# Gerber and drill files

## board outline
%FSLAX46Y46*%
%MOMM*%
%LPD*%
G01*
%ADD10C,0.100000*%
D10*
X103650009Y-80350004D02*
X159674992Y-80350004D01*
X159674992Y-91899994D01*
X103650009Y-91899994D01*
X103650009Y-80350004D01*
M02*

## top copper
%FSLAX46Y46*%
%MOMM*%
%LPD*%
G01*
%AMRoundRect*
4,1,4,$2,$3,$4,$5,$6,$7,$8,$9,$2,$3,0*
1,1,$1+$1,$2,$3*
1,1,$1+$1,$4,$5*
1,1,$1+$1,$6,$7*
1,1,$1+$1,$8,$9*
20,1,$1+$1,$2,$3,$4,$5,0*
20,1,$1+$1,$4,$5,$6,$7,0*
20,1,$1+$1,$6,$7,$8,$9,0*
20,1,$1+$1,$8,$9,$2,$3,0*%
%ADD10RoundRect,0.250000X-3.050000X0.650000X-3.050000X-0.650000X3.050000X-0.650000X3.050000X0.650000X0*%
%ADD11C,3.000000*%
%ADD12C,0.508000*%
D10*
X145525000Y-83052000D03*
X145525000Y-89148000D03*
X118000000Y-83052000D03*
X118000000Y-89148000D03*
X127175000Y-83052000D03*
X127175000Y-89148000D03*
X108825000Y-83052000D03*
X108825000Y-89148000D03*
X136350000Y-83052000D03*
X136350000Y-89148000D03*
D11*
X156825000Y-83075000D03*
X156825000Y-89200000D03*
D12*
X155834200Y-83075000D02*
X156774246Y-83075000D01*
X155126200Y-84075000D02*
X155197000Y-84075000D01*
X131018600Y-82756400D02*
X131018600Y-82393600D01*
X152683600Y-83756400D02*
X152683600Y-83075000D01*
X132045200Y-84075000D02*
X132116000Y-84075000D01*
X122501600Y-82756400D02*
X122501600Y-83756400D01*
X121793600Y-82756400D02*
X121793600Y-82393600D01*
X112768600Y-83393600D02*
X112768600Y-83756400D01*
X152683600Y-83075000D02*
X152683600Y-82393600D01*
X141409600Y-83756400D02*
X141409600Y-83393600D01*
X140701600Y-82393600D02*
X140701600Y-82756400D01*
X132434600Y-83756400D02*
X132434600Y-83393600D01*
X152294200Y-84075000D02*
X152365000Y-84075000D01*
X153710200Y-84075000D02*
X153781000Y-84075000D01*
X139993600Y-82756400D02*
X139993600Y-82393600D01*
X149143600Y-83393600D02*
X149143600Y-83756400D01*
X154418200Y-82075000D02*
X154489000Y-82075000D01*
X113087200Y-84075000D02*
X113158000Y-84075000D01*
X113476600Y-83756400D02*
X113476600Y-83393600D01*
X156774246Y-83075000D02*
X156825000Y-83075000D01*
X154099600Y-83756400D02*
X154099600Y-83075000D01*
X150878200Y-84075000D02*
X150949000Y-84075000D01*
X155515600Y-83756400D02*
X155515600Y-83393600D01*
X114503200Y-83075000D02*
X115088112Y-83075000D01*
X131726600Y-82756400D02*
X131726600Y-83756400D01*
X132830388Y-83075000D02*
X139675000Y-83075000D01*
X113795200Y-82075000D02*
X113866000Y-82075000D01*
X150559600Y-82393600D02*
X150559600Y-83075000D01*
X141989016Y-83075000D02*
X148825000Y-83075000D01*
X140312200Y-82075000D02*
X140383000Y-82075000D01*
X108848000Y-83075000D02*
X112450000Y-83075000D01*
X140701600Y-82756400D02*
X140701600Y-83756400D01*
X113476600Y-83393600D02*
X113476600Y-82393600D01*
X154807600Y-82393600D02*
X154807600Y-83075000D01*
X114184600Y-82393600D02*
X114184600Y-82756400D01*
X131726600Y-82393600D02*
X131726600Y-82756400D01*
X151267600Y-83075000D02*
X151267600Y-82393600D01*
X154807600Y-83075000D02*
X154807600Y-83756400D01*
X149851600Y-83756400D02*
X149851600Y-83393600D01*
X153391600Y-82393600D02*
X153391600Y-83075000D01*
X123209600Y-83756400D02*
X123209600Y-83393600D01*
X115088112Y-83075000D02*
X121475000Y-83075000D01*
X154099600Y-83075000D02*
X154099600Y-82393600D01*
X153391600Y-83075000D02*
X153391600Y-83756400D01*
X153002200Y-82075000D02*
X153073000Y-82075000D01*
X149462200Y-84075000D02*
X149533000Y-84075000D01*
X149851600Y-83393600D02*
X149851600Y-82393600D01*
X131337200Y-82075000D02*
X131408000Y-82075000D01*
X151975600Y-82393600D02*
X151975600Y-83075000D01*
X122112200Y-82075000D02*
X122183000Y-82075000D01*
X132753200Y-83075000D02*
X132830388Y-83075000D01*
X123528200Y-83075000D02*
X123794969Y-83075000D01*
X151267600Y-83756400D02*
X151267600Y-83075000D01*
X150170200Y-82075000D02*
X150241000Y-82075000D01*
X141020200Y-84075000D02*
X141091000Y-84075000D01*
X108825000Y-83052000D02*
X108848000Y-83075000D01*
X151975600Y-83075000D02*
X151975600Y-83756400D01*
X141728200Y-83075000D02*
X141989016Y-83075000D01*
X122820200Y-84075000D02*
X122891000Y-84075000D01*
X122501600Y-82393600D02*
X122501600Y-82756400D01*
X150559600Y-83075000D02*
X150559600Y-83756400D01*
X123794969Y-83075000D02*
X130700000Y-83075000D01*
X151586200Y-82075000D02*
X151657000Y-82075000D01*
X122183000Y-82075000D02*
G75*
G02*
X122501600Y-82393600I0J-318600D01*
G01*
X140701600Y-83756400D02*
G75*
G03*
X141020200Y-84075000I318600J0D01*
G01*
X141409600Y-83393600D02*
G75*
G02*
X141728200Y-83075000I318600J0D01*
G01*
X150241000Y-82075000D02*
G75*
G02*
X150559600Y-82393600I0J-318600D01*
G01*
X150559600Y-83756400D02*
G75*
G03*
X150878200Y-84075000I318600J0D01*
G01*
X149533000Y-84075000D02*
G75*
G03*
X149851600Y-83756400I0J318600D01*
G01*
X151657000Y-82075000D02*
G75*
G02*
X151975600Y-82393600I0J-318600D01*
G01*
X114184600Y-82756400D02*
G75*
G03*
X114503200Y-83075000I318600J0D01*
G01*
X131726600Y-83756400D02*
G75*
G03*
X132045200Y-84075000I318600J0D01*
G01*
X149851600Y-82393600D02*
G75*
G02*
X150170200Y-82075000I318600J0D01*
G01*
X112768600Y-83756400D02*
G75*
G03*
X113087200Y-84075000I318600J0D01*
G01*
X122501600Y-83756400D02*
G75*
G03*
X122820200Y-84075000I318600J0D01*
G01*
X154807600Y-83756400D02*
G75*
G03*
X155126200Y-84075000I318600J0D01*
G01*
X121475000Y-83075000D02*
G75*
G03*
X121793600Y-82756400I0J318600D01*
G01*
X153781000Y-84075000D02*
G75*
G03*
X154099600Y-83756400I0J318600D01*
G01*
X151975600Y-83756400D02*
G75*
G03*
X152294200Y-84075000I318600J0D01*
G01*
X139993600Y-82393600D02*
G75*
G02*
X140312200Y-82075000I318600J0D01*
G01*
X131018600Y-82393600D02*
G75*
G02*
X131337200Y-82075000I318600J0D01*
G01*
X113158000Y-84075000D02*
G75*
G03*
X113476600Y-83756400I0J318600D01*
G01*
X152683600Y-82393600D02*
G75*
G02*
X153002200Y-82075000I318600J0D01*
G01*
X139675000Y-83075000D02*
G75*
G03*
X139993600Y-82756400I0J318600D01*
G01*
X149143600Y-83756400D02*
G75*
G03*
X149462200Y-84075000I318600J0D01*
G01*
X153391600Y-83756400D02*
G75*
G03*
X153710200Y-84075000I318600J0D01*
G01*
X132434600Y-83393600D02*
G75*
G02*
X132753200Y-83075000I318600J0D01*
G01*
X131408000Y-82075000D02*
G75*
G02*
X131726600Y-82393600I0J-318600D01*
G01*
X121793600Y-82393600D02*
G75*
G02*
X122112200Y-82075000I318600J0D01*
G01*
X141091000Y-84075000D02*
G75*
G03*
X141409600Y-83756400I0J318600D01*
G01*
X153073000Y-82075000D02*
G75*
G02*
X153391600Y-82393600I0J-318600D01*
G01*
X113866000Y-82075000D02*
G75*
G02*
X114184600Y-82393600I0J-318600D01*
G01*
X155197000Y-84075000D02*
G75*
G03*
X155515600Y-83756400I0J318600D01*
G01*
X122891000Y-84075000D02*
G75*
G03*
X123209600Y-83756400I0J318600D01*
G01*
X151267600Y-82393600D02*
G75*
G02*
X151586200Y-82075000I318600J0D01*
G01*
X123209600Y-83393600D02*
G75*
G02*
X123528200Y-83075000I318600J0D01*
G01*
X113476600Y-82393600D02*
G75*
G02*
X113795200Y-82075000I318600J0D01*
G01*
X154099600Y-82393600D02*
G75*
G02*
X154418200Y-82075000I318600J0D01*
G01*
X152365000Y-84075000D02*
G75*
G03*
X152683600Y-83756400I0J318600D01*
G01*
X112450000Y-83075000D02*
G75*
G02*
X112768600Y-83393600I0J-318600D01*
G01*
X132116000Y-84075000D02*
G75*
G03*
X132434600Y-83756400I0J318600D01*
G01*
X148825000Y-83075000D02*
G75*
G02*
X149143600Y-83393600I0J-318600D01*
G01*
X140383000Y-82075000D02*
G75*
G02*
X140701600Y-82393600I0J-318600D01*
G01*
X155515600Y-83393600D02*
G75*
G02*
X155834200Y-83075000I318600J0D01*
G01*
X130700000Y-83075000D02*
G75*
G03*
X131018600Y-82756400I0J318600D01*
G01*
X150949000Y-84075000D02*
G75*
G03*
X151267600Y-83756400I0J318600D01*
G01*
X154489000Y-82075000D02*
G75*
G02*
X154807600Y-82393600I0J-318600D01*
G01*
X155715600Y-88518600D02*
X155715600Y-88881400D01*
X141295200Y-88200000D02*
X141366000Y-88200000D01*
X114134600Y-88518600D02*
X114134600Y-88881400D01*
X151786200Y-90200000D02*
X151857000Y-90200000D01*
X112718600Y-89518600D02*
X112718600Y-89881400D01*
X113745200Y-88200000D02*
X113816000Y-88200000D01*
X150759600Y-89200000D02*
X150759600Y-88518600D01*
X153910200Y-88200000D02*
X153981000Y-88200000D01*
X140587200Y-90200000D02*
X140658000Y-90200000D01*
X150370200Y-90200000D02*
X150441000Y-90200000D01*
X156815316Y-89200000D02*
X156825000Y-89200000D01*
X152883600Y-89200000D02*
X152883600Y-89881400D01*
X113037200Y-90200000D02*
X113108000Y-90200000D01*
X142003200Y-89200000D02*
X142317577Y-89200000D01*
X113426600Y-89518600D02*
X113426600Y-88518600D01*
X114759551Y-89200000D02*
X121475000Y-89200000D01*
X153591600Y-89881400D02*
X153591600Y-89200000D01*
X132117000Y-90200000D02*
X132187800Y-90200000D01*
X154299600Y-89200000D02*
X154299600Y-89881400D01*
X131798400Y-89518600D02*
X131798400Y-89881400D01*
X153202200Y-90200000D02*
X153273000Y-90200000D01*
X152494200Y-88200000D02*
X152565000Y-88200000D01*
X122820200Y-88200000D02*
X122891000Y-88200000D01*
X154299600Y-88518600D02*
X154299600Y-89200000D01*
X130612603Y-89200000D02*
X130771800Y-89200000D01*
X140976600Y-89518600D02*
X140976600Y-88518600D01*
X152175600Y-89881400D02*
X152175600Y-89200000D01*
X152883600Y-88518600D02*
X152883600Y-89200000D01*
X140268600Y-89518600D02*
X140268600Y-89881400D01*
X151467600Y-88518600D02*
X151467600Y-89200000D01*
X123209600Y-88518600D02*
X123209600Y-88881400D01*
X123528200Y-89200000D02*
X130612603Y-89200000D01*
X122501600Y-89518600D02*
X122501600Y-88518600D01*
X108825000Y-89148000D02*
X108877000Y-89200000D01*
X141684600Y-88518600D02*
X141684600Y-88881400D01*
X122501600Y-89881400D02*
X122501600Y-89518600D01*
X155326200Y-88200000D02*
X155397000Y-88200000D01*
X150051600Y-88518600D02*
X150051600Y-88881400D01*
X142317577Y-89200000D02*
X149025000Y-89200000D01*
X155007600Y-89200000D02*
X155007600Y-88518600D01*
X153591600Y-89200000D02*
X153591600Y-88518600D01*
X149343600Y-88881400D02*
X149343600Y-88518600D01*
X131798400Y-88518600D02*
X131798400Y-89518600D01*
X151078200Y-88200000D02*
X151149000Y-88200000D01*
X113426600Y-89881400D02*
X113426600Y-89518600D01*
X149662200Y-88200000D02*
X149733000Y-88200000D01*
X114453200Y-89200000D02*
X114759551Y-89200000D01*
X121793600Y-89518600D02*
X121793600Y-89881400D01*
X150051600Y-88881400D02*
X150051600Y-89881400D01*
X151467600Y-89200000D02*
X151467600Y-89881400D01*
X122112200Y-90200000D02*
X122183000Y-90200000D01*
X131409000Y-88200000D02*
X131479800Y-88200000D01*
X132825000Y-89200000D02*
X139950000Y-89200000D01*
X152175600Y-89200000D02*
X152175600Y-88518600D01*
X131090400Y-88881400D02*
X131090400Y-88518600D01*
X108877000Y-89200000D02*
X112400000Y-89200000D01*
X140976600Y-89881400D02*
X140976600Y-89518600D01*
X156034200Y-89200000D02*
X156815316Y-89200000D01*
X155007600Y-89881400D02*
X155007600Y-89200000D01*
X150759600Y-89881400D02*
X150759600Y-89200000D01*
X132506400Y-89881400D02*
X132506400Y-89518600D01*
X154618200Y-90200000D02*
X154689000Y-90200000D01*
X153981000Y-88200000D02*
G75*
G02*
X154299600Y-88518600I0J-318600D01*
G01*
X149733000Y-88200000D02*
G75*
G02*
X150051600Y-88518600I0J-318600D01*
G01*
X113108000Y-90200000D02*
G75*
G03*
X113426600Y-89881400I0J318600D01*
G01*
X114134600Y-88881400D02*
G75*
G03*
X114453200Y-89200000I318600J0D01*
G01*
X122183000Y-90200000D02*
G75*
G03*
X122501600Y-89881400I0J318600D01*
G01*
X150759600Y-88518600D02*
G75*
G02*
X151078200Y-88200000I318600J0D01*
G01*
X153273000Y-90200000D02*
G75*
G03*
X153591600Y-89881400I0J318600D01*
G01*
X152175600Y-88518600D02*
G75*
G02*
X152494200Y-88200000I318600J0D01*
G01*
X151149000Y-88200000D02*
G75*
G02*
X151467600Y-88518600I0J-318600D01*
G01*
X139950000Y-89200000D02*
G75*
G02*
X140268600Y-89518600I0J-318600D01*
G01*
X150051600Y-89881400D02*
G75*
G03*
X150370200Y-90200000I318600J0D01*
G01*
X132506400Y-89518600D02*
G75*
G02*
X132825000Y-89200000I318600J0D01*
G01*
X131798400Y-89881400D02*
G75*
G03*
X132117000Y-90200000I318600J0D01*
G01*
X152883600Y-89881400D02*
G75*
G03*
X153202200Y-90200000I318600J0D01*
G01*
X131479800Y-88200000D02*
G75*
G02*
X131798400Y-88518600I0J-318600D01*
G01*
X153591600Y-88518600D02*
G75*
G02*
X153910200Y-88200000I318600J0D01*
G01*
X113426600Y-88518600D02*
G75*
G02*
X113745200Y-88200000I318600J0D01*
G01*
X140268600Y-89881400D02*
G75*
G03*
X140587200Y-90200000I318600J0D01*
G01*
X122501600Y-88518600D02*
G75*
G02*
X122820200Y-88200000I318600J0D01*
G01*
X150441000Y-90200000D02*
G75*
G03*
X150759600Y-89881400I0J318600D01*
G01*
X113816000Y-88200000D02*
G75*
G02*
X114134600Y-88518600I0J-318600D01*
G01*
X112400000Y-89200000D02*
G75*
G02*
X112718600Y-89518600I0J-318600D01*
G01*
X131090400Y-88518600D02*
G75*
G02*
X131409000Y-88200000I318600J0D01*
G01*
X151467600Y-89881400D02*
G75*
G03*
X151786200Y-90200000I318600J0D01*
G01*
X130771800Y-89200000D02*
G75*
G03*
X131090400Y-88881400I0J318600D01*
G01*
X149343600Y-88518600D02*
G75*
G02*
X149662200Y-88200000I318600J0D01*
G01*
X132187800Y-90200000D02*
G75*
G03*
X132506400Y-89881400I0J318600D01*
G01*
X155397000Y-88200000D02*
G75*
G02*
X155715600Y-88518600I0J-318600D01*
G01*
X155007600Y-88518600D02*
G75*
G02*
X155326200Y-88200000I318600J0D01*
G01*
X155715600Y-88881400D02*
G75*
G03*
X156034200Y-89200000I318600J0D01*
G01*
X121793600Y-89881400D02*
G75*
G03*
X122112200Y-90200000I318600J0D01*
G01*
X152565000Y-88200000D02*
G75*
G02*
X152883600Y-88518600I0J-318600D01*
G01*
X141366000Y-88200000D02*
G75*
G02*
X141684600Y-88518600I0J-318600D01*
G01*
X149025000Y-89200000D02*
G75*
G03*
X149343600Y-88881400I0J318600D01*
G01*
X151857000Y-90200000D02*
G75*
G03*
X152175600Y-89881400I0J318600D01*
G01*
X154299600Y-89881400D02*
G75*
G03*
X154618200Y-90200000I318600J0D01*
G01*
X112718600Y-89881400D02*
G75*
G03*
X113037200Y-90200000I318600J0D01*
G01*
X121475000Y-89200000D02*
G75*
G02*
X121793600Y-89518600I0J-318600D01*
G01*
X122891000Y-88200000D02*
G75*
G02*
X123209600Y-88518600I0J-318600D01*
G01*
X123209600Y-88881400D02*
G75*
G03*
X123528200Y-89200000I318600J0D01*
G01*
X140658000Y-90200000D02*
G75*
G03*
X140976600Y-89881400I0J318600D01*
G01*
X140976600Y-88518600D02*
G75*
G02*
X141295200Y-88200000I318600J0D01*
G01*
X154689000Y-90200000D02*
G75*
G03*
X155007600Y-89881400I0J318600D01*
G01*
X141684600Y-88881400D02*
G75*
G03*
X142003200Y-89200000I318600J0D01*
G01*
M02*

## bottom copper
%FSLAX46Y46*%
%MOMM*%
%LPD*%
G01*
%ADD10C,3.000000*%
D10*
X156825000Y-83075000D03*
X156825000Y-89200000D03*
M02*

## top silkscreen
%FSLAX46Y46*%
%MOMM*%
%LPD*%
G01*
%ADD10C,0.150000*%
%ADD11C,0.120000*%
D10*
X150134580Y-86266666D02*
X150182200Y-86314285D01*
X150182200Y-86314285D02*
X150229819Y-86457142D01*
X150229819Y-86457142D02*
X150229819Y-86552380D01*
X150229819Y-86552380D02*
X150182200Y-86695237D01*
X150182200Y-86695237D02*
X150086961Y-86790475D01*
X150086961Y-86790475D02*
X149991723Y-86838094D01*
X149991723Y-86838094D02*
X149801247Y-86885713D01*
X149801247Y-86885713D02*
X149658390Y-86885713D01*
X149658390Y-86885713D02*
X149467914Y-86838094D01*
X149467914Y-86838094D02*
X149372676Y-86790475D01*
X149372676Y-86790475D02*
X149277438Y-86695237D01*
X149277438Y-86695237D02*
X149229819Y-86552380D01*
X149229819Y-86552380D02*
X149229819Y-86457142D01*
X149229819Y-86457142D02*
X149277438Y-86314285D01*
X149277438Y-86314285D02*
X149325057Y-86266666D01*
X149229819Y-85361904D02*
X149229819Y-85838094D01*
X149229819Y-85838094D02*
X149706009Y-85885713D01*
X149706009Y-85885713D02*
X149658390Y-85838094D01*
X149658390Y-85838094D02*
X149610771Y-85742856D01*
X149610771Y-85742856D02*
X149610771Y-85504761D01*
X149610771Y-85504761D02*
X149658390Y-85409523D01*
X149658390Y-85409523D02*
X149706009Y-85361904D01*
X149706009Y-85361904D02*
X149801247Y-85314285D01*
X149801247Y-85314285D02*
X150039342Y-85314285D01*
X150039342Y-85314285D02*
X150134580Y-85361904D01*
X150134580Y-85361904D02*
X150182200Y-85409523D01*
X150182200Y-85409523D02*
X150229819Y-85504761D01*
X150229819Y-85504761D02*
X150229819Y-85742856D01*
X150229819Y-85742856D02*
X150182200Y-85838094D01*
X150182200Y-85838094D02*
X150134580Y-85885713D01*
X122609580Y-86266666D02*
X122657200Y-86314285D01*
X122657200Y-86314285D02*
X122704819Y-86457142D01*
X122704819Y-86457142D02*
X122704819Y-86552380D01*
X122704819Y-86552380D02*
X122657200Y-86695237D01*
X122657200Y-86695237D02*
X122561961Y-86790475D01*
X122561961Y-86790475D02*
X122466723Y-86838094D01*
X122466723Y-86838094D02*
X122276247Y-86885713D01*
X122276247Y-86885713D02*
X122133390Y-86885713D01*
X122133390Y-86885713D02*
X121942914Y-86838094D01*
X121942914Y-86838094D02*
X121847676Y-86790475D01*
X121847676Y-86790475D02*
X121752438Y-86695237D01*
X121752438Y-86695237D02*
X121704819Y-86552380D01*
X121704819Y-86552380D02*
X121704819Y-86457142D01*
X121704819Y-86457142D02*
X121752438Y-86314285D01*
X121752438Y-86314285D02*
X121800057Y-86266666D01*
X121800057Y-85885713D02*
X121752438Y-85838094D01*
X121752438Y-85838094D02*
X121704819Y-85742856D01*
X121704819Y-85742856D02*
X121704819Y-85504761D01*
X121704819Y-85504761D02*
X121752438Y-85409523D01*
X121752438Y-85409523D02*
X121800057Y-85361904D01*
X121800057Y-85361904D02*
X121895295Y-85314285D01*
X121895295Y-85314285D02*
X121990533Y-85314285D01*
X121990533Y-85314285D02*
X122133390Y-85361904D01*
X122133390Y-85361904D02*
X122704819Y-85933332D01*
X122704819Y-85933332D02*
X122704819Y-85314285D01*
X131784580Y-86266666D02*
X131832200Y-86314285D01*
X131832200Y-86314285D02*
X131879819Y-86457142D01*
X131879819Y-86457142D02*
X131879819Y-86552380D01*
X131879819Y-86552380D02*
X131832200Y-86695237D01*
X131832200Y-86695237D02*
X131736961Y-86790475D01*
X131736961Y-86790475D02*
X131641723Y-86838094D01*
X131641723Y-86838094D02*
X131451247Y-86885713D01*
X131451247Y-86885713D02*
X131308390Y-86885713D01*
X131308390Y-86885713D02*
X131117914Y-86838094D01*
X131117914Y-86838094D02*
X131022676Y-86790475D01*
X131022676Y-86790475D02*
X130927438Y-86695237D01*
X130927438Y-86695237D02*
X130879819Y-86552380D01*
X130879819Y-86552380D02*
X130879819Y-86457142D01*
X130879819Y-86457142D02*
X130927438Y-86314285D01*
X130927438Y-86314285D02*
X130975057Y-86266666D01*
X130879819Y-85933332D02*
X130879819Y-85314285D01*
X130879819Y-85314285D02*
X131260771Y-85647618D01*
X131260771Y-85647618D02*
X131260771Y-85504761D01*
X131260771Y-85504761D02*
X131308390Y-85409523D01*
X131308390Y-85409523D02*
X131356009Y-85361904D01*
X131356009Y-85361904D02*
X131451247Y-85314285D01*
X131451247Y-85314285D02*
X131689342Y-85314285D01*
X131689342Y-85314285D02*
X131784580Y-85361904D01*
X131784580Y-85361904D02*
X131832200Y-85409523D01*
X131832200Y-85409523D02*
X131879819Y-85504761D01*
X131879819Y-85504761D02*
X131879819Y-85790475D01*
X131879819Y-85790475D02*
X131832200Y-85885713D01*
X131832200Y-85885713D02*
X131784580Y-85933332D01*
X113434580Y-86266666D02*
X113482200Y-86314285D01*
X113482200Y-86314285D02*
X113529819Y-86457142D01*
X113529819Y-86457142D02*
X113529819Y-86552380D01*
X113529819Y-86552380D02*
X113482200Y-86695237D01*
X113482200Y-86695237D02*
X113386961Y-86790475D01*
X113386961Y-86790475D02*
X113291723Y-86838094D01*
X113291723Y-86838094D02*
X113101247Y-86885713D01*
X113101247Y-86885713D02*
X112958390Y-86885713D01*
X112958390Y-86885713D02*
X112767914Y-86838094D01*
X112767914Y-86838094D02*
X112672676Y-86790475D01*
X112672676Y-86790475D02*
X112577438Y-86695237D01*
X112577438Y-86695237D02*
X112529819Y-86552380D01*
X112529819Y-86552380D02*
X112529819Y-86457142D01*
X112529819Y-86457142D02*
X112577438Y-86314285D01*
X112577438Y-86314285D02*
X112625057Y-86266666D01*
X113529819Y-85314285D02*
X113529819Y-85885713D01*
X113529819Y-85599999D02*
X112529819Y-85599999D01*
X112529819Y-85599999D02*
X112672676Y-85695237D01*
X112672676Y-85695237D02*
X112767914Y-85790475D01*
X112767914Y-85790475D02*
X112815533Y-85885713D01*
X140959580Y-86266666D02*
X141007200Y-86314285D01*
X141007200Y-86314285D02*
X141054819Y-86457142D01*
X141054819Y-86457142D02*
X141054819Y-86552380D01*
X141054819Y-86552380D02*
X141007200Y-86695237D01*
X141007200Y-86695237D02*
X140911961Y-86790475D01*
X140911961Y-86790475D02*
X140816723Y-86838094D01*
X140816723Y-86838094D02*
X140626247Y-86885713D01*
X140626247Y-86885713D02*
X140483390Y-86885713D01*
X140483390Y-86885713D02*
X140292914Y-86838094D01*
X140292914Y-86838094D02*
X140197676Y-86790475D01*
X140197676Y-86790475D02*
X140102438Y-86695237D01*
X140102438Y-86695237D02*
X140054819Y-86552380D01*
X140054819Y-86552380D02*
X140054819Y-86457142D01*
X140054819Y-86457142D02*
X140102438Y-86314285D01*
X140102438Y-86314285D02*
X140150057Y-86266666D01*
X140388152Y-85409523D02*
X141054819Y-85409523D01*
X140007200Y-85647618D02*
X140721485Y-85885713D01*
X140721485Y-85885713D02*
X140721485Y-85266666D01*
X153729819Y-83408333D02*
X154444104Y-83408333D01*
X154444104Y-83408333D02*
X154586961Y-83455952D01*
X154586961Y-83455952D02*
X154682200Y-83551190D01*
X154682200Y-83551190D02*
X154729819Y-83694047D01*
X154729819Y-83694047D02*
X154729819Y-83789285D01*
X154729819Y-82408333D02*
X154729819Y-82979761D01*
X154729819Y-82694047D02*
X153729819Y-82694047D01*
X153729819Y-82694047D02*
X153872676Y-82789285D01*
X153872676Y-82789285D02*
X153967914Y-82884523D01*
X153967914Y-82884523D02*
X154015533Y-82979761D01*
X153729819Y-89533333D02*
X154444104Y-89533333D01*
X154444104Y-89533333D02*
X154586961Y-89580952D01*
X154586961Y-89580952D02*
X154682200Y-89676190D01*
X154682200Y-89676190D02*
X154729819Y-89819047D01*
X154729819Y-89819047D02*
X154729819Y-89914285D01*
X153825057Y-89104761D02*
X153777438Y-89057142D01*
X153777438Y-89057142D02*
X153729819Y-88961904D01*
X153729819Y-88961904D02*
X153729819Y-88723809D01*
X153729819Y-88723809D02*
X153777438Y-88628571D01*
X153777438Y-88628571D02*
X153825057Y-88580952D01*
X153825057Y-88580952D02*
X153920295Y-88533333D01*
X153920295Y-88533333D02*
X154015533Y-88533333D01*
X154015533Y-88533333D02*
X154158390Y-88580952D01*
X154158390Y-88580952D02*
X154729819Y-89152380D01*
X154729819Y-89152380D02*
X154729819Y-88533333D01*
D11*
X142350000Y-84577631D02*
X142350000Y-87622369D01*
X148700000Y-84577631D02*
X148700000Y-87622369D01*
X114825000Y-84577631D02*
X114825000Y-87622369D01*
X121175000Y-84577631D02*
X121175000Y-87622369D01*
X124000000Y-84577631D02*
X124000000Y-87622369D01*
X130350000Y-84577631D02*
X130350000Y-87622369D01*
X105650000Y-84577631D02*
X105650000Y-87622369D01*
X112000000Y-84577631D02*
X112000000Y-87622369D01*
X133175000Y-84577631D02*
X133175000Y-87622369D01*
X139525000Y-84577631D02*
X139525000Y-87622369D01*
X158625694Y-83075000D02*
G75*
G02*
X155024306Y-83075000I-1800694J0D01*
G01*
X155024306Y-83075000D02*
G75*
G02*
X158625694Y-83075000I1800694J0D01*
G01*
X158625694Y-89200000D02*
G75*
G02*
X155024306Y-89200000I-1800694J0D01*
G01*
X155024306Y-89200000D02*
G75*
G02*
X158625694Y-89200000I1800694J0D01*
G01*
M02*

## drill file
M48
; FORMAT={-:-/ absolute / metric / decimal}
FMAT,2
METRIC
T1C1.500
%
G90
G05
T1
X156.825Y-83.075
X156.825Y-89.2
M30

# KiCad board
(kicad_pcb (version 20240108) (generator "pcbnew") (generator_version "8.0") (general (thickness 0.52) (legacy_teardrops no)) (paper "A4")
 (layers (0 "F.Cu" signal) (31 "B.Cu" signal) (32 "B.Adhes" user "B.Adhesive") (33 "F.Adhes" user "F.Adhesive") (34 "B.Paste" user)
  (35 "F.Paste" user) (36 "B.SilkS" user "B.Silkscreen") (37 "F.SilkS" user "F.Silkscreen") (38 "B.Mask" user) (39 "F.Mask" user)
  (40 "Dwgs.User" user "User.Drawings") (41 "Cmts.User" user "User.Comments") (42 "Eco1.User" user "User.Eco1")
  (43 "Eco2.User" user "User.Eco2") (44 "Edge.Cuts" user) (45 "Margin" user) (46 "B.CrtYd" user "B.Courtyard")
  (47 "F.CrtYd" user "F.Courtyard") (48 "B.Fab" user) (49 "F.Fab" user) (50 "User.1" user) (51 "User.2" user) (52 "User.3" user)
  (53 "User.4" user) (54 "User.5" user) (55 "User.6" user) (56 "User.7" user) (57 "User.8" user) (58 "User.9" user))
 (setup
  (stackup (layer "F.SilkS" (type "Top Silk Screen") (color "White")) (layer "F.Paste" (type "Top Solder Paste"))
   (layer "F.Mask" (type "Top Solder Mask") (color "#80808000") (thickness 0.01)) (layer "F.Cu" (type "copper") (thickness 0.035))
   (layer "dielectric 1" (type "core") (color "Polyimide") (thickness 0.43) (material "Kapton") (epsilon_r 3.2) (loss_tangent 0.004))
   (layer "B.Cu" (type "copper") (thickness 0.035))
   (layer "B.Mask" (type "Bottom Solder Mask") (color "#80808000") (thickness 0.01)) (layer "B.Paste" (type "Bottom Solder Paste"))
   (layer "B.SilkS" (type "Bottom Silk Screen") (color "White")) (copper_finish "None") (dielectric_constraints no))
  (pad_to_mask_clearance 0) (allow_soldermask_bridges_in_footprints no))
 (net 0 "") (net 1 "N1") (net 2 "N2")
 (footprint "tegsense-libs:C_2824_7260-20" (layer "F.Cu") (at 145.525 86.1 -90)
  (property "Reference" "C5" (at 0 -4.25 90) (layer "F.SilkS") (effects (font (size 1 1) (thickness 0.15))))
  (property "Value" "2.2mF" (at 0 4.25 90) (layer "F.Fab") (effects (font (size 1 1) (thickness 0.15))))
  (fp_line (start -1.522369 3.175) (end 1.522369 3.175) (stroke (width 0.12) (type solid)) (layer "F.SilkS"))
  (fp_line (start -1.522369 -3.175) (end 1.522369 -3.175) (stroke (width 0.12) (type solid)) (layer "F.SilkS"))
  (pad "1" smd roundrect (at -3.048 0 270) (size 1.8 6.6) (layers "F.Cu" "F.Paste" "F.Mask") (roundrect_rratio 0.138889) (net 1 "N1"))
  (pad "2" smd roundrect (at 3.048 0 270) (size 1.8 6.6) (layers "F.Cu" "F.Paste" "F.Mask") (roundrect_rratio 0.138889) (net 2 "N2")))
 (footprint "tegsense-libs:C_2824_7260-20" (layer "F.Cu") (at 118 86.1 -90)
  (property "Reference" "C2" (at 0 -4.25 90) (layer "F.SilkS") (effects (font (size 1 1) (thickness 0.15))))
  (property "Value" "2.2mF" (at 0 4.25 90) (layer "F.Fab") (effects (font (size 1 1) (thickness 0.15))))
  (fp_line (start -1.522369 3.175) (end 1.522369 3.175) (stroke (width 0.12) (type solid)) (layer "F.SilkS"))
  (fp_line (start -1.522369 -3.175) (end 1.522369 -3.175) (stroke (width 0.12) (type solid)) (layer "F.SilkS"))
  (pad "1" smd roundrect (at -3.048 0 270) (size 1.8 6.6) (layers "F.Cu" "F.Paste" "F.Mask") (roundrect_rratio 0.138889) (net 1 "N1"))
  (pad "2" smd roundrect (at 3.048 0 270) (size 1.8 6.6) (layers "F.Cu" "F.Paste" "F.Mask") (roundrect_rratio 0.138889) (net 2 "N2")))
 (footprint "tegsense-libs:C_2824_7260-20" (layer "F.Cu") (at 127.175 86.1 -90)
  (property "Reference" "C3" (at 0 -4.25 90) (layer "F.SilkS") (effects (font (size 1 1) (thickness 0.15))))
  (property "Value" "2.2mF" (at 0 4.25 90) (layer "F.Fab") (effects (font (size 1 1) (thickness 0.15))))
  (fp_line (start -1.522369 3.175) (end 1.522369 3.175) (stroke (width 0.12) (type solid)) (layer "F.SilkS"))
  (fp_line (start -1.522369 -3.175) (end 1.522369 -3.175) (stroke (width 0.12) (type solid)) (layer "F.SilkS"))
  (pad "1" smd roundrect (at -3.048 0 270) (size 1.8 6.6) (layers "F.Cu" "F.Paste" "F.Mask") (roundrect_rratio 0.138889) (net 1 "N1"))
  (pad "2" smd roundrect (at 3.048 0 270) (size 1.8 6.6) (layers "F.Cu" "F.Paste" "F.Mask") (roundrect_rratio 0.138889) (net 2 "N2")))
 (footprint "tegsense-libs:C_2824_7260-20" (layer "F.Cu") (at 108.825 86.1 -90)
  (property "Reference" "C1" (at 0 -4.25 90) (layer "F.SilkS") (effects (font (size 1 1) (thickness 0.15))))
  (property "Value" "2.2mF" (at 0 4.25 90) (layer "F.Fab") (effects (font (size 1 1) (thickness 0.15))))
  (fp_line (start -1.522369 3.175) (end 1.522369 3.175) (stroke (width 0.12) (type solid)) (layer "F.SilkS"))
  (fp_line (start -1.522369 -3.175) (end 1.522369 -3.175) (stroke (width 0.12) (type solid)) (layer "F.SilkS"))
  (pad "1" smd roundrect (at -3.048 0 270) (size 1.8 6.6) (layers "F.Cu" "F.Paste" "F.Mask") (roundrect_rratio 0.138889) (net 1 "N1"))
  (pad "2" smd roundrect (at 3.048 0 270) (size 1.8 6.6) (layers "F.Cu" "F.Paste" "F.Mask") (roundrect_rratio 0.138889) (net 2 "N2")))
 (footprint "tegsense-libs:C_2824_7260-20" (layer "F.Cu") (at 136.35 86.1 -90)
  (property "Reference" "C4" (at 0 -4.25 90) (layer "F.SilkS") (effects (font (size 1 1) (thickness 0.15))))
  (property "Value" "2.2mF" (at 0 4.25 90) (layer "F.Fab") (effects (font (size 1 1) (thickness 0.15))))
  (fp_line (start -1.522369 3.175) (end 1.522369 3.175) (stroke (width 0.12) (type solid)) (layer "F.SilkS"))
  (fp_line (start -1.522369 -3.175) (end 1.522369 -3.175) (stroke (width 0.12) (type solid)) (layer "F.SilkS"))
  (pad "1" smd roundrect (at -3.048 0 270) (size 1.8 6.6) (layers "F.Cu" "F.Paste" "F.Mask") (roundrect_rratio 0.138889) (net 1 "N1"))
  (pad "2" smd roundrect (at 3.048 0 270) (size 1.8 6.6) (layers "F.Cu" "F.Paste" "F.Mask") (roundrect_rratio 0.138889) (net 2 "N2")))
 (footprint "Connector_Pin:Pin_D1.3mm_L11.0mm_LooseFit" (layer "F.Cu") (at 156.825 83.075 -90)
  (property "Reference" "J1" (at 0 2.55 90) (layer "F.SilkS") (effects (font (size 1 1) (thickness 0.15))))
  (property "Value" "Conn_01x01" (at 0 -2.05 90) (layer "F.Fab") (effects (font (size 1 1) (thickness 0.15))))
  (fp_circle (center 0 0) (end 1.8 0.05) (stroke (width 0.12) (type solid)) (fill none) (layer "F.SilkS"))
  (pad "1" thru_hole circle (at 0 0 270) (size 3 3) (drill 1.5) (layers "*.Cu" "*.Mask") (remove_unused_layers no) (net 1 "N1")))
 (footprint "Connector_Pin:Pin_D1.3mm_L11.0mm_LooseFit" (layer "F.Cu") (at 156.825 89.2 -90)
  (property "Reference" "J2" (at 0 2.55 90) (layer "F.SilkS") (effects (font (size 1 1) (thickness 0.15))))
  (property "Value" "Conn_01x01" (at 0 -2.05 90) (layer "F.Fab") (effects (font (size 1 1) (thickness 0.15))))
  (fp_circle (center 0 0) (end 1.8 0.05) (stroke (width 0.12) (type solid)) (fill none) (layer "F.SilkS"))
  (pad "1" thru_hole circle (at 0 0 270) (size 3 3) (drill 1.5) (layers "*.Cu" "*.Mask") (remove_unused_layers no) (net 2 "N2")))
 (gr_rect (start 103.650009 80.350004) (end 159.674992 91.899994) (stroke (width 0.1) (type solid)) (fill none) (layer "Edge.Cuts"))
 (segment (start 155.8342 83.075) (end 156.774246 83.075) (width 0.508) (layer "F.Cu") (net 1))
 (segment (start 155.1262 84.075) (end 155.197 84.075) (width 0.508) (layer "F.Cu") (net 1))
 (segment (start 131.0186 82.7564) (end 131.0186 82.3936) (width 0.508) (layer "F.Cu") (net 1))
 (segment (start 152.6836 83.7564) (end 152.6836 83.075) (width 0.508) (layer "F.Cu") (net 1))
 (segment (start 132.0452 84.075) (end 132.116 84.075) (width 0.508) (layer "F.Cu") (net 1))
 (segment (start 122.5016 82.7564) (end 122.5016 83.7564) (width 0.508) (layer "F.Cu") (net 1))
 (segment (start 121.7936 82.7564) (end 121.7936 82.3936) (width 0.508) (layer "F.Cu") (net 1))
 (segment (start 112.7686 83.3936) (end 112.7686 83.7564) (width 0.508) (layer "F.Cu") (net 1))
 (segment (start 152.6836 83.075) (end 152.6836 82.3936) (width 0.508) (layer "F.Cu") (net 1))
 (segment (start 141.4096 83.7564) (end 141.4096 83.3936) (width 0.508) (layer "F.Cu") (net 1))
 (segment (start 140.7016 82.3936) (end 140.7016 82.7564) (width 0.508) (layer "F.Cu") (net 1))
 (segment (start 132.4346 83.7564) (end 132.4346 83.3936) (width 0.508) (layer "F.Cu") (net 1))
 (segment (start 152.2942 84.075) (end 152.365 84.075) (width 0.508) (layer "F.Cu") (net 1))
 (segment (start 153.7102 84.075) (end 153.781 84.075) (width 0.508) (layer "F.Cu") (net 1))
 (segment (start 139.9936 82.7564) (end 139.9936 82.3936) (width 0.508) (layer "F.Cu") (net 1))
 (segment (start 149.1436 83.3936) (end 149.1436 83.7564) (width 0.508) (layer "F.Cu") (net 1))
 (segment (start 154.4182 82.075) (end 154.489 82.075) (width 0.508) (layer "F.Cu") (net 1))
 (segment (start 113.0872 84.075) (end 113.158 84.075) (width 0.508) (layer "F.Cu") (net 1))
 (segment (start 113.4766 83.7564) (end 113.4766 83.3936) (width 0.508) (layer "F.Cu") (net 1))
 (segment (start 156.774246 83.075) (end 156.825 83.075) (width 0.508) (layer "F.Cu") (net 1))
 (segment (start 154.0996 83.7564) (end 154.0996 83.075) (width 0.508) (layer "F.Cu") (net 1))
 (segment (start 150.8782 84.075) (end 150.949 84.075) (width 0.508) (layer "F.Cu") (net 1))
 (segment (start 155.5156 83.7564) (end 155.5156 83.3936) (width 0.508) (layer "F.Cu") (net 1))
 (segment (start 114.5032 83.075) (end 115.088112 83.075) (width 0.508) (layer "F.Cu") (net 1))
 (segment (start 131.7266 82.7564) (end 131.7266 83.7564) (width 0.508) (layer "F.Cu") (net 1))
 (segment (start 132.830388 83.075) (end 139.675 83.075) (width 0.508) (layer "F.Cu") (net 1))
 (segment (start 113.7952 82.075) (end 113.866 82.075) (width 0.508) (layer "F.Cu") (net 1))
 (segment (start 150.5596 82.3936) (end 150.5596 83.075) (width 0.508) (layer "F.Cu") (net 1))
 (segment (start 141.989016 83.075) (end 148.825 83.075) (width 0.508) (layer "F.Cu") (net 1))
 (segment (start 140.3122 82.075) (end 140.383 82.075) (width 0.508) (layer "F.Cu") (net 1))
 (segment (start 108.848 83.075) (end 112.45 83.075) (width 0.508) (layer "F.Cu") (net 1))
 (segment (start 140.7016 82.7564) (end 140.7016 83.7564) (width 0.508) (layer "F.Cu") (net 1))
 (segment (start 113.4766 83.3936) (end 113.4766 82.3936) (width 0.508) (layer "F.Cu") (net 1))
 (segment (start 154.8076 82.3936) (end 154.8076 83.075) (width 0.508) (layer "F.Cu") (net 1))
 (segment (start 114.1846 82.3936) (end 114.1846 82.7564) (width 0.508) (layer "F.Cu") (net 1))
 (segment (start 131.7266 82.3936) (end 131.7266 82.7564) (width 0.508) (layer "F.Cu") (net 1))
 (segment (start 151.2676 83.075) (end 151.2676 82.3936) (width 0.508) (layer "F.Cu") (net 1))
 (segment (start 154.8076 83.075) (end 154.8076 83.7564) (width 0.508) (layer "F.Cu") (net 1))
 (segment (start 149.8516 83.7564) (end 149.8516 83.3936) (width 0.508) (layer "F.Cu") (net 1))
 (segment (start 153.3916 82.3936) (end 153.3916 83.075) (width 0.508) (layer "F.Cu") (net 1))
 (segment (start 123.2096 83.7564) (end 123.2096 83.3936) (width 0.508) (layer "F.Cu") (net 1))
 (segment (start 115.088112 83.075) (end 121.475 83.075) (width 0.508) (layer "F.Cu") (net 1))
 (segment (start 154.0996 83.075) (end 154.0996 82.3936) (width 0.508) (layer "F.Cu") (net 1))
 (segment (start 153.3916 83.075) (end 153.3916 83.7564) (width 0.508) (layer "F.Cu") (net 1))
 (segment (start 153.0022 82.075) (end 153.073 82.075) (width 0.508) (layer "F.Cu") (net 1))
 (segment (start 149.4622 84.075) (end 149.533 84.075) (width 0.508) (layer "F.Cu") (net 1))
 (segment (start 149.8516 83.3936) (end 149.8516 82.3936) (width 0.508) (layer "F.Cu") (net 1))
 (segment (start 131.3372 82.075) (end 131.408 82.075) (width 0.508) (layer "F.Cu") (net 1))
 (segment (start 151.9756 82.3936) (end 151.9756 83.075) (width 0.508) (layer "F.Cu") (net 1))
 (segment (start 122.1122 82.075) (end 122.183 82.075) (width 0.508) (layer "F.Cu") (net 1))
 (segment (start 132.7532 83.075) (end 132.830388 83.075) (width 0.508) (layer "F.Cu") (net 1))
 (segment (start 123.5282 83.075) (end 123.794969 83.075) (width 0.508) (layer "F.Cu") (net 1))
 (segment (start 151.2676 83.7564) (end 151.2676 83.075) (width 0.508) (layer "F.Cu") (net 1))
 (segment (start 150.1702 82.075) (end 150.241 82.075) (width 0.508) (layer "F.Cu") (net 1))
 (segment (start 141.0202 84.075) (end 141.091 84.075) (width 0.508) (layer "F.Cu") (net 1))
 (segment (start 108.825 83.052) (end 108.848 83.075) (width 0.508) (layer "F.Cu") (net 1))
 (segment (start 151.9756 83.075) (end 151.9756 83.7564) (width 0.508) (layer "F.Cu") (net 1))
 (segment (start 141.7282 83.075) (end 141.989016 83.075) (width 0.508) (layer "F.Cu") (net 1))
 (segment (start 122.8202 84.075) (end 122.891 84.075) (width 0.508) (layer "F.Cu") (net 1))
 (segment (start 122.5016 82.3936) (end 122.5016 82.7564) (width 0.508) (layer "F.Cu") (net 1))
 (segment (start 150.5596 83.075) (end 150.5596 83.7564) (width 0.508) (layer "F.Cu") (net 1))
 (segment (start 123.794969 83.075) (end 130.7 83.075) (width 0.508) (layer "F.Cu") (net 1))
 (segment (start 151.5862 82.075) (end 151.657 82.075) (width 0.508) (layer "F.Cu") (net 1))
 (arc (start 122.183 82.075) (mid 122.408284 82.168316) (end 122.5016 82.3936) (width 0.508) (layer "F.Cu") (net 1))
 (arc (start 140.7016 83.7564) (mid 140.794916 83.981684) (end 141.0202 84.075) (width 0.508) (layer "F.Cu") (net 1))
 (arc (start 141.4096 83.3936) (mid 141.502916 83.168316) (end 141.7282 83.075) (width 0.508) (layer "F.Cu") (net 1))
 (arc (start 150.241 82.075) (mid 150.466284 82.168316) (end 150.5596 82.3936) (width 0.508) (layer "F.Cu") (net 1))
 (arc (start 150.5596 83.7564) (mid 150.652916 83.981684) (end 150.8782 84.075) (width 0.508) (layer "F.Cu") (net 1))
 (arc (start 149.533 84.075) (mid 149.758284 83.981684) (end 149.8516 83.7564) (width 0.508) (layer "F.Cu") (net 1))
 (arc (start 151.657 82.075) (mid 151.882284 82.168316) (end 151.9756 82.3936) (width 0.508) (layer "F.Cu") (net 1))
 (arc (start 114.1846 82.7564) (mid 114.277916 82.981684) (end 114.5032 83.075) (width 0.508) (layer "F.Cu") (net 1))
 (arc (start 131.7266 83.7564) (mid 131.819916 83.981684) (end 132.0452 84.075) (width 0.508) (layer "F.Cu") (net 1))
 (arc (start 149.8516 82.3936) (mid 149.944916 82.168316) (end 150.1702 82.075) (width 0.508) (layer "F.Cu") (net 1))
 (arc (start 112.7686 83.7564) (mid 112.861916 83.981684) (end 113.0872 84.075) (width 0.508) (layer "F.Cu") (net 1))
 (arc (start 122.5016 83.7564) (mid 122.594916 83.981684) (end 122.8202 84.075) (width 0.508) (layer "F.Cu") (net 1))
 (arc (start 154.8076 83.7564) (mid 154.900916 83.981684) (end 155.1262 84.075) (width 0.508) (layer "F.Cu") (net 1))
 (arc (start 121.475 83.075) (mid 121.700284 82.981684) (end 121.7936 82.7564) (width 0.508) (layer "F.Cu") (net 1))
 (arc (start 153.781 84.075) (mid 154.006284 83.981684) (end 154.0996 83.7564) (width 0.508) (layer "F.Cu") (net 1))
 (arc (start 151.9756 83.7564) (mid 152.068916 83.981684) (end 152.2942 84.075) (width 0.508) (layer "F.Cu") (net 1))
 (arc (start 139.9936 82.3936) (mid 140.086916 82.168316) (end 140.3122 82.075) (width 0.508) (layer "F.Cu") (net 1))
 (arc (start 131.0186 82.3936) (mid 131.111916 82.168316) (end 131.3372 82.075) (width 0.508) (layer "F.Cu") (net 1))
 (arc (start 113.158 84.075) (mid 113.383284 83.981684) (end 113.4766 83.7564) (width 0.508) (layer "F.Cu") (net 1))
 (arc (start 152.6836 82.3936) (mid 152.776916 82.168316) (end 153.0022 82.075) (width 0.508) (layer "F.Cu") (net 1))
 (arc (start 139.675 83.075) (mid 139.900284 82.981684) (end 139.9936 82.7564) (width 0.508) (layer "F.Cu") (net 1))
 (arc (start 149.1436 83.7564) (mid 149.236916 83.981684) (end 149.4622 84.075) (width 0.508) (layer "F.Cu") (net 1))
 (arc (start 153.3916 83.7564) (mid 153.484916 83.981684) (end 153.7102 84.075) (width 0.508) (layer "F.Cu") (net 1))
 (arc (start 132.4346 83.3936) (mid 132.527916 83.168316) (end 132.7532 83.075) (width 0.508) (layer "F.Cu") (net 1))
 (arc (start 131.408 82.075) (mid 131.633284 82.168316) (end 131.7266 82.3936) (width 0.508) (layer "F.Cu") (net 1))
 (arc (start 121.7936 82.3936) (mid 121.886916 82.168316) (end 122.1122 82.075) (width 0.508) (layer "F.Cu") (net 1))
 (arc (start 141.091 84.075) (mid 141.316284 83.981684) (end 141.4096 83.7564) (width 0.508) (layer "F.Cu") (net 1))
 (arc (start 153.073 82.075) (mid 153.298284 82.168316) (end 153.3916 82.3936) (width 0.508) (layer "F.Cu") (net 1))
 (arc (start 113.866 82.075) (mid 114.091284 82.168316) (end 114.1846 82.3936) (width 0.508) (layer "F.Cu") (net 1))
 (arc (start 155.197 84.075) (mid 155.422284 83.981684) (end 155.5156 83.7564) (width 0.508) (layer "F.Cu") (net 1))
 (arc (start 122.891 84.075) (mid 123.116284 83.981684) (end 123.2096 83.7564) (width 0.508) (layer "F.Cu") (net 1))
 (arc (start 151.2676 82.3936) (mid 151.360916 82.168316) (end 151.5862 82.075) (width 0.508) (layer "F.Cu") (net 1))
 (arc (start 123.2096 83.3936) (mid 123.302916 83.168316) (end 123.5282 83.075) (width 0.508) (layer "F.Cu") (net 1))
 (arc (start 113.4766 82.3936) (mid 113.569916 82.168316) (end 113.7952 82.075) (width 0.508) (layer "F.Cu") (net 1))
 (arc (start 154.0996 82.3936) (mid 154.192916 82.168316) (end 154.4182 82.075) (width 0.508) (layer "F.Cu") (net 1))
 (arc (start 152.365 84.075) (mid 152.590284 83.981684) (end 152.6836 83.7564) (width 0.508) (layer "F.Cu") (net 1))
 (arc (start 112.45 83.075) (mid 112.675284 83.168316) (end 112.7686 83.3936) (width 0.508) (layer "F.Cu") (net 1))
 (arc (start 132.116 84.075) (mid 132.341284 83.981684) (end 132.4346 83.7564) (width 0.508) (layer "F.Cu") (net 1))
 (arc (start 148.825 83.075) (mid 149.050284 83.168316) (end 149.1436 83.3936) (width 0.508) (layer "F.Cu") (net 1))
 (arc (start 140.383 82.075) (mid 140.608284 82.168316) (end 140.7016 82.3936) (width 0.508) (layer "F.Cu") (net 1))
 (arc (start 155.5156 83.3936) (mid 155.608916 83.168316) (end 155.8342 83.075) (width 0.508) (layer "F.Cu") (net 1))
 (arc (start 130.7 83.075) (mid 130.925284 82.981684) (end 131.0186 82.7564) (width 0.508) (layer "F.Cu") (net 1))
 (arc (start 150.949 84.075) (mid 151.174284 83.981684) (end 151.2676 83.7564) (width 0.508) (layer "F.Cu") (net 1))
 (arc (start 154.489 82.075) (mid 154.714284 82.168316) (end 154.8076 82.3936) (width 0.508) (layer "F.Cu") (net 1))
 (segment (start 155.7156 88.5186) (end 155.7156 88.8814) (width 0.508) (layer "F.Cu") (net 2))
 (segment (start 141.2952 88.2) (end 141.366 88.2) (width 0.508) (layer "F.Cu") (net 2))
 (segment (start 114.1346 88.5186) (end 114.1346 88.8814) (width 0.508) (layer "F.Cu") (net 2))
 (segment (start 151.7862 90.2) (end 151.857 90.2) (width 0.508) (layer "F.Cu") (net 2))
 (segment (start 112.7186 89.5186) (end 112.7186 89.8814) (width 0.508) (layer "F.Cu") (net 2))
 (segment (start 113.7452 88.2) (end 113.816 88.2) (width 0.508) (layer "F.Cu") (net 2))
 (segment (start 150.7596 89.2) (end 150.7596 88.5186) (width 0.508) (layer "F.Cu") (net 2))
 (segment (start 153.9102 88.2) (end 153.981 88.2) (width 0.508) (layer "F.Cu") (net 2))
 (segment (start 140.5872 90.2) (end 140.658 90.2) (width 0.508) (layer "F.Cu") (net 2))
 (segment (start 150.3702 90.2) (end 150.441 90.2) (width 0.508) (layer "F.Cu") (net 2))
 (segment (start 156.815316 89.2) (end 156.825 89.2) (width 0.508) (layer "F.Cu") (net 2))
 (segment (start 152.8836 89.2) (end 152.8836 89.8814) (width 0.508) (layer "F.Cu") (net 2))
 (segment (start 113.0372 90.2) (end 113.108 90.2) (width 0.508) (layer "F.Cu") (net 2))
 (segment (start 142.0032 89.2) (end 142.317577 89.2) (width 0.508) (layer "F.Cu") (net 2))
 (segment (start 113.4266 89.5186) (end 113.4266 88.5186) (width 0.508) (layer "F.Cu") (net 2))
 (segment (start 114.759551 89.2) (end 121.475 89.2) (width 0.508) (layer "F.Cu") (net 2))
 (segment (start 153.5916 89.8814) (end 153.5916 89.2) (width 0.508) (layer "F.Cu") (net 2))
 (segment (start 132.117 90.2) (end 132.1878 90.2) (width 0.508) (layer "F.Cu") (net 2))
 (segment (start 154.2996 89.2) (end 154.2996 89.8814) (width 0.508) (layer "F.Cu") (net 2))
 (segment (start 131.7984 89.5186) (end 131.7984 89.8814) (width 0.508) (layer "F.Cu") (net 2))
 (segment (start 153.2022 90.2) (end 153.273 90.2) (width 0.508) (layer "F.Cu") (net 2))
 (segment (start 152.4942 88.2) (end 152.565 88.2) (width 0.508) (layer "F.Cu") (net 2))
 (segment (start 122.8202 88.2) (end 122.891 88.2) (width 0.508) (layer "F.Cu") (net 2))
 (segment (start 154.2996 88.5186) (end 154.2996 89.2) (width 0.508) (layer "F.Cu") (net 2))
 (segment (start 130.612603 89.2) (end 130.7718 89.2) (width 0.508) (layer "F.Cu") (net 2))
 (segment (start 140.9766 89.5186) (end 140.9766 88.5186) (width 0.508) (layer "F.Cu") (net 2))
 (segment (start 152.1756 89.8814) (end 152.1756 89.2) (width 0.508) (layer "F.Cu") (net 2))
 (segment (start 152.8836 88.5186) (end 152.8836 89.2) (width 0.508) (layer "F.Cu") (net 2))
 (segment (start 140.2686 89.5186) (end 140.2686 89.8814) (width 0.508) (layer "F.Cu") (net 2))
 (segment (start 151.4676 88.5186) (end 151.4676 89.2) (width 0.508) (layer "F.Cu") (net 2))
 (segment (start 123.2096 88.5186) (end 123.2096 88.8814) (width 0.508) (layer "F.Cu") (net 2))
 (segment (start 123.5282 89.2) (end 130.612603 89.2) (width 0.508) (layer "F.Cu") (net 2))
 (segment (start 122.5016 89.5186) (end 122.5016 88.5186) (width 0.508) (layer "F.Cu") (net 2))
 (segment (start 108.825 89.148) (end 108.877 89.2) (width 0.508) (layer "F.Cu") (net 2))
 (segment (start 141.6846 88.5186) (end 141.6846 88.8814) (width 0.508) (layer "F.Cu") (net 2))
 (segment (start 122.5016 89.8814) (end 122.5016 89.5186) (width 0.508) (layer "F.Cu") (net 2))
 (segment (start 155.3262 88.2) (end 155.397 88.2) (width 0.508) (layer "F.Cu") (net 2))
 (segment (start 150.0516 88.5186) (end 150.0516 88.8814) (width 0.508) (layer "F.Cu") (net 2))
 (segment (start 142.317577 89.2) (end 149.025 89.2) (width 0.508) (layer "F.Cu") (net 2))
 (segment (start 155.0076 89.2) (end 155.0076 88.5186) (width 0.508) (layer "F.Cu") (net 2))
 (segment (start 153.5916 89.2) (end 153.5916 88.5186) (width 0.508) (layer "F.Cu") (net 2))
 (segment (start 149.3436 88.8814) (end 149.3436 88.5186) (width 0.508) (layer "F.Cu") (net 2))
 (segment (start 131.7984 88.5186) (end 131.7984 89.5186) (width 0.508) (layer "F.Cu") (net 2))
 (segment (start 151.0782 88.2) (end 151.149 88.2) (width 0.508) (layer "F.Cu") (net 2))
 (segment (start 113.4266 89.8814) (end 113.4266 89.5186) (width 0.508) (layer "F.Cu") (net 2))
 (segment (start 149.6622 88.2) (end 149.733 88.2) (width 0.508) (layer "F.Cu") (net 2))
 (segment (start 114.4532 89.2) (end 114.759551 89.2) (width 0.508) (layer "F.Cu") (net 2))
 (segment (start 121.7936 89.5186) (end 121.7936 89.8814) (width 0.508) (layer "F.Cu") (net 2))
 (segment (start 150.0516 88.8814) (end 150.0516 89.8814) (width 0.508) (layer "F.Cu") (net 2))
 (segment (start 151.4676 89.2) (end 151.4676 89.8814) (width 0.508) (layer "F.Cu") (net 2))
 (segment (start 122.1122 90.2) (end 122.183 90.2) (width 0.508) (layer "F.Cu") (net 2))
 (segment (start 131.409 88.2) (end 131.4798 88.2) (width 0.508) (layer "F.Cu") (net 2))
 (segment (start 132.825 89.2) (end 139.95 89.2) (width 0.508) (layer "F.Cu") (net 2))
 (segment (start 152.1756 89.2) (end 152.1756 88.5186) (width 0.508) (layer "F.Cu") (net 2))
 (segment (start 131.0904 88.8814) (end 131.0904 88.5186) (width 0.508) (layer "F.Cu") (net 2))
 (segment (start 108.877 89.2) (end 112.4 89.2) (width 0.508) (layer "F.Cu") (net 2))
 (segment (start 140.9766 89.8814) (end 140.9766 89.5186) (width 0.508) (layer "F.Cu") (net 2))
 (segment (start 156.0342 89.2) (end 156.815316 89.2) (width 0.508) (layer "F.Cu") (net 2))
 (segment (start 155.0076 89.8814) (end 155.0076 89.2) (width 0.508) (layer "F.Cu") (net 2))
 (segment (start 150.7596 89.8814) (end 150.7596 89.2) (width 0.508) (layer "F.Cu") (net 2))
 (segment (start 132.5064 89.8814) (end 132.5064 89.5186) (width 0.508) (layer "F.Cu") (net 2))
 (segment (start 154.6182 90.2) (end 154.689 90.2) (width 0.508) (layer "F.Cu") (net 2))
 (arc (start 153.981 88.2) (mid 154.206284 88.293316) (end 154.2996 88.5186) (width 0.508) (layer "F.Cu") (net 2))
 (arc (start 149.733 88.2) (mid 149.958284 88.293316) (end 150.0516 88.5186) (width 0.508) (layer "F.Cu") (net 2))
 (arc (start 113.108 90.2) (mid 113.333284 90.106684) (end 113.4266 89.8814) (width 0.508) (layer "F.Cu") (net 2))
 (arc (start 114.1346 88.8814) (mid 114.227916 89.106684) (end 114.4532 89.2) (width 0.508) (layer "F.Cu") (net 2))
 (arc (start 122.183 90.2) (mid 122.408284 90.106684) (end 122.5016 89.8814) (width 0.508) (layer "F.Cu") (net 2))
 (arc (start 150.7596 88.5186) (mid 150.852916 88.293316) (end 151.0782 88.2) (width 0.508) (layer "F.Cu") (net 2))
 (arc (start 153.273 90.2) (mid 153.498284 90.106684) (end 153.5916 89.8814) (width 0.508) (layer "F.Cu") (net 2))
 (arc (start 152.1756 88.5186) (mid 152.268916 88.293316) (end 152.4942 88.2) (width 0.508) (layer "F.Cu") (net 2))
 (arc (start 151.149 88.2) (mid 151.374284 88.293316) (end 151.4676 88.5186) (width 0.508) (layer "F.Cu") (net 2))
 (arc (start 139.95 89.2) (mid 140.175284 89.293316) (end 140.2686 89.5186) (width 0.508) (layer "F.Cu") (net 2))
 (arc (start 150.0516 89.8814) (mid 150.144916 90.106684) (end 150.3702 90.2) (width 0.508) (layer "F.Cu") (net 2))
 (arc (start 132.5064 89.5186) (mid 132.599716 89.293316) (end 132.825 89.2) (width 0.508) (layer "F.Cu") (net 2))
 (arc (start 131.7984 89.8814) (mid 131.891716 90.106684) (end 132.117 90.2) (width 0.508) (layer "F.Cu") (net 2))
 (arc (start 152.8836 89.8814) (mid 152.976916 90.106684) (end 153.2022 90.2) (width 0.508) (layer "F.Cu") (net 2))
 (arc (start 131.4798 88.2) (mid 131.705084 88.293316) (end 131.7984 88.5186) (width 0.508) (layer "F.Cu") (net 2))
 (arc (start 153.5916 88.5186) (mid 153.684916 88.293316) (end 153.9102 88.2) (width 0.508) (layer "F.Cu") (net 2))
 (arc (start 113.4266 88.5186) (mid 113.519916 88.293316) (end 113.7452 88.2) (width 0.508) (layer "F.Cu") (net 2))
 (arc (start 140.2686 89.8814) (mid 140.361916 90.106684) (end 140.5872 90.2) (width 0.508) (layer "F.Cu") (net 2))
 (arc (start 122.5016 88.5186) (mid 122.594916 88.293316) (end 122.8202 88.2) (width 0.508) (layer "F.Cu") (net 2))
 (arc (start 150.441 90.2) (mid 150.666284 90.106684) (end 150.7596 89.8814) (width 0.508) (layer "F.Cu") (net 2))
 (arc (start 113.816 88.2) (mid 114.041284 88.293316) (end 114.1346 88.5186) (width 0.508) (layer "F.Cu") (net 2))
 (arc (start 112.4 89.2) (mid 112.625284 89.293316) (end 112.7186 89.5186) (width 0.508) (layer "F.Cu") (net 2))
 (arc (start 131.0904 88.5186) (mid 131.183716 88.293316) (end 131.409 88.2) (width 0.508) (layer "F.Cu") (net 2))
 (arc (start 151.4676 89.8814) (mid 151.560916 90.106684) (end 151.7862 90.2) (width 0.508) (layer "F.Cu") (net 2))
 (arc (start 130.7718 89.2) (mid 130.997084 89.106684) (end 131.0904 88.8814) (width 0.508) (layer "F.Cu") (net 2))
 (arc (start 149.3436 88.5186) (mid 149.436916 88.293316) (end 149.6622 88.2) (width 0.508) (layer "F.Cu") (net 2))
 (arc (start 132.1878 90.2) (mid 132.413084 90.106684) (end 132.5064 89.8814) (width 0.508) (layer "F.Cu") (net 2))
 (arc (start 155.397 88.2) (mid 155.622284 88.293316) (end 155.7156 88.5186) (width 0.508) (layer "F.Cu") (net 2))
 (arc (start 155.0076 88.5186) (mid 155.100916 88.293316) (end 155.3262 88.2) (width 0.508) (layer "F.Cu") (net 2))
 (arc (start 155.7156 88.8814) (mid 155.808916 89.106684) (end 156.0342 89.2) (width 0.508) (layer "F.Cu") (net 2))
 (arc (start 121.7936 89.8814) (mid 121.886916 90.106684) (end 122.1122 90.2) (width 0.508) (layer "F.Cu") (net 2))
 (arc (start 152.565 88.2) (mid 152.790284 88.293316) (end 152.8836 88.5186) (width 0.508) (layer "F.Cu") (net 2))
 (arc (start 141.366 88.2) (mid 141.591284 88.293316) (end 141.6846 88.5186) (width 0.508) (layer "F.Cu") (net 2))
 (arc (start 149.025 89.2) (mid 149.250284 89.106684) (end 149.3436 88.8814) (width 0.508) (layer "F.Cu") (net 2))
 (arc (start 151.857 90.2) (mid 152.082284 90.106684) (end 152.1756 89.8814) (width 0.508) (layer "F.Cu") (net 2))
 (arc (start 154.2996 89.8814) (mid 154.392916 90.106684) (end 154.6182 90.2) (width 0.508) (layer "F.Cu") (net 2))
 (arc (start 112.7186 89.8814) (mid 112.811916 90.106684) (end 113.0372 90.2) (width 0.508) (layer "F.Cu") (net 2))
 (arc (start 121.475 89.2) (mid 121.700284 89.293316) (end 121.7936 89.5186) (width 0.508) (layer "F.Cu") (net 2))
 (arc (start 122.891 88.2) (mid 123.116284 88.293316) (end 123.2096 88.5186) (width 0.508) (layer "F.Cu") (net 2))
 (arc (start 123.2096 88.8814) (mid 123.302916 89.106684) (end 123.5282 89.2) (width 0.508) (layer "F.Cu") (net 2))
 (arc (start 140.658 90.2) (mid 140.883284 90.106684) (end 140.9766 89.8814) (width 0.508) (layer "F.Cu") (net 2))
 (arc (start 140.9766 88.5186) (mid 141.069916 88.293316) (end 141.2952 88.2) (width 0.508) (layer "F.Cu") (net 2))
 (arc (start 154.689 90.2) (mid 154.914284 90.106684) (end 155.0076 89.8814) (width 0.508) (layer "F.Cu") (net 2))
 (arc (start 141.6846 88.8814) (mid 141.777916 89.106684) (end 142.0032 89.2) (width 0.508) (layer "F.Cu") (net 2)))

